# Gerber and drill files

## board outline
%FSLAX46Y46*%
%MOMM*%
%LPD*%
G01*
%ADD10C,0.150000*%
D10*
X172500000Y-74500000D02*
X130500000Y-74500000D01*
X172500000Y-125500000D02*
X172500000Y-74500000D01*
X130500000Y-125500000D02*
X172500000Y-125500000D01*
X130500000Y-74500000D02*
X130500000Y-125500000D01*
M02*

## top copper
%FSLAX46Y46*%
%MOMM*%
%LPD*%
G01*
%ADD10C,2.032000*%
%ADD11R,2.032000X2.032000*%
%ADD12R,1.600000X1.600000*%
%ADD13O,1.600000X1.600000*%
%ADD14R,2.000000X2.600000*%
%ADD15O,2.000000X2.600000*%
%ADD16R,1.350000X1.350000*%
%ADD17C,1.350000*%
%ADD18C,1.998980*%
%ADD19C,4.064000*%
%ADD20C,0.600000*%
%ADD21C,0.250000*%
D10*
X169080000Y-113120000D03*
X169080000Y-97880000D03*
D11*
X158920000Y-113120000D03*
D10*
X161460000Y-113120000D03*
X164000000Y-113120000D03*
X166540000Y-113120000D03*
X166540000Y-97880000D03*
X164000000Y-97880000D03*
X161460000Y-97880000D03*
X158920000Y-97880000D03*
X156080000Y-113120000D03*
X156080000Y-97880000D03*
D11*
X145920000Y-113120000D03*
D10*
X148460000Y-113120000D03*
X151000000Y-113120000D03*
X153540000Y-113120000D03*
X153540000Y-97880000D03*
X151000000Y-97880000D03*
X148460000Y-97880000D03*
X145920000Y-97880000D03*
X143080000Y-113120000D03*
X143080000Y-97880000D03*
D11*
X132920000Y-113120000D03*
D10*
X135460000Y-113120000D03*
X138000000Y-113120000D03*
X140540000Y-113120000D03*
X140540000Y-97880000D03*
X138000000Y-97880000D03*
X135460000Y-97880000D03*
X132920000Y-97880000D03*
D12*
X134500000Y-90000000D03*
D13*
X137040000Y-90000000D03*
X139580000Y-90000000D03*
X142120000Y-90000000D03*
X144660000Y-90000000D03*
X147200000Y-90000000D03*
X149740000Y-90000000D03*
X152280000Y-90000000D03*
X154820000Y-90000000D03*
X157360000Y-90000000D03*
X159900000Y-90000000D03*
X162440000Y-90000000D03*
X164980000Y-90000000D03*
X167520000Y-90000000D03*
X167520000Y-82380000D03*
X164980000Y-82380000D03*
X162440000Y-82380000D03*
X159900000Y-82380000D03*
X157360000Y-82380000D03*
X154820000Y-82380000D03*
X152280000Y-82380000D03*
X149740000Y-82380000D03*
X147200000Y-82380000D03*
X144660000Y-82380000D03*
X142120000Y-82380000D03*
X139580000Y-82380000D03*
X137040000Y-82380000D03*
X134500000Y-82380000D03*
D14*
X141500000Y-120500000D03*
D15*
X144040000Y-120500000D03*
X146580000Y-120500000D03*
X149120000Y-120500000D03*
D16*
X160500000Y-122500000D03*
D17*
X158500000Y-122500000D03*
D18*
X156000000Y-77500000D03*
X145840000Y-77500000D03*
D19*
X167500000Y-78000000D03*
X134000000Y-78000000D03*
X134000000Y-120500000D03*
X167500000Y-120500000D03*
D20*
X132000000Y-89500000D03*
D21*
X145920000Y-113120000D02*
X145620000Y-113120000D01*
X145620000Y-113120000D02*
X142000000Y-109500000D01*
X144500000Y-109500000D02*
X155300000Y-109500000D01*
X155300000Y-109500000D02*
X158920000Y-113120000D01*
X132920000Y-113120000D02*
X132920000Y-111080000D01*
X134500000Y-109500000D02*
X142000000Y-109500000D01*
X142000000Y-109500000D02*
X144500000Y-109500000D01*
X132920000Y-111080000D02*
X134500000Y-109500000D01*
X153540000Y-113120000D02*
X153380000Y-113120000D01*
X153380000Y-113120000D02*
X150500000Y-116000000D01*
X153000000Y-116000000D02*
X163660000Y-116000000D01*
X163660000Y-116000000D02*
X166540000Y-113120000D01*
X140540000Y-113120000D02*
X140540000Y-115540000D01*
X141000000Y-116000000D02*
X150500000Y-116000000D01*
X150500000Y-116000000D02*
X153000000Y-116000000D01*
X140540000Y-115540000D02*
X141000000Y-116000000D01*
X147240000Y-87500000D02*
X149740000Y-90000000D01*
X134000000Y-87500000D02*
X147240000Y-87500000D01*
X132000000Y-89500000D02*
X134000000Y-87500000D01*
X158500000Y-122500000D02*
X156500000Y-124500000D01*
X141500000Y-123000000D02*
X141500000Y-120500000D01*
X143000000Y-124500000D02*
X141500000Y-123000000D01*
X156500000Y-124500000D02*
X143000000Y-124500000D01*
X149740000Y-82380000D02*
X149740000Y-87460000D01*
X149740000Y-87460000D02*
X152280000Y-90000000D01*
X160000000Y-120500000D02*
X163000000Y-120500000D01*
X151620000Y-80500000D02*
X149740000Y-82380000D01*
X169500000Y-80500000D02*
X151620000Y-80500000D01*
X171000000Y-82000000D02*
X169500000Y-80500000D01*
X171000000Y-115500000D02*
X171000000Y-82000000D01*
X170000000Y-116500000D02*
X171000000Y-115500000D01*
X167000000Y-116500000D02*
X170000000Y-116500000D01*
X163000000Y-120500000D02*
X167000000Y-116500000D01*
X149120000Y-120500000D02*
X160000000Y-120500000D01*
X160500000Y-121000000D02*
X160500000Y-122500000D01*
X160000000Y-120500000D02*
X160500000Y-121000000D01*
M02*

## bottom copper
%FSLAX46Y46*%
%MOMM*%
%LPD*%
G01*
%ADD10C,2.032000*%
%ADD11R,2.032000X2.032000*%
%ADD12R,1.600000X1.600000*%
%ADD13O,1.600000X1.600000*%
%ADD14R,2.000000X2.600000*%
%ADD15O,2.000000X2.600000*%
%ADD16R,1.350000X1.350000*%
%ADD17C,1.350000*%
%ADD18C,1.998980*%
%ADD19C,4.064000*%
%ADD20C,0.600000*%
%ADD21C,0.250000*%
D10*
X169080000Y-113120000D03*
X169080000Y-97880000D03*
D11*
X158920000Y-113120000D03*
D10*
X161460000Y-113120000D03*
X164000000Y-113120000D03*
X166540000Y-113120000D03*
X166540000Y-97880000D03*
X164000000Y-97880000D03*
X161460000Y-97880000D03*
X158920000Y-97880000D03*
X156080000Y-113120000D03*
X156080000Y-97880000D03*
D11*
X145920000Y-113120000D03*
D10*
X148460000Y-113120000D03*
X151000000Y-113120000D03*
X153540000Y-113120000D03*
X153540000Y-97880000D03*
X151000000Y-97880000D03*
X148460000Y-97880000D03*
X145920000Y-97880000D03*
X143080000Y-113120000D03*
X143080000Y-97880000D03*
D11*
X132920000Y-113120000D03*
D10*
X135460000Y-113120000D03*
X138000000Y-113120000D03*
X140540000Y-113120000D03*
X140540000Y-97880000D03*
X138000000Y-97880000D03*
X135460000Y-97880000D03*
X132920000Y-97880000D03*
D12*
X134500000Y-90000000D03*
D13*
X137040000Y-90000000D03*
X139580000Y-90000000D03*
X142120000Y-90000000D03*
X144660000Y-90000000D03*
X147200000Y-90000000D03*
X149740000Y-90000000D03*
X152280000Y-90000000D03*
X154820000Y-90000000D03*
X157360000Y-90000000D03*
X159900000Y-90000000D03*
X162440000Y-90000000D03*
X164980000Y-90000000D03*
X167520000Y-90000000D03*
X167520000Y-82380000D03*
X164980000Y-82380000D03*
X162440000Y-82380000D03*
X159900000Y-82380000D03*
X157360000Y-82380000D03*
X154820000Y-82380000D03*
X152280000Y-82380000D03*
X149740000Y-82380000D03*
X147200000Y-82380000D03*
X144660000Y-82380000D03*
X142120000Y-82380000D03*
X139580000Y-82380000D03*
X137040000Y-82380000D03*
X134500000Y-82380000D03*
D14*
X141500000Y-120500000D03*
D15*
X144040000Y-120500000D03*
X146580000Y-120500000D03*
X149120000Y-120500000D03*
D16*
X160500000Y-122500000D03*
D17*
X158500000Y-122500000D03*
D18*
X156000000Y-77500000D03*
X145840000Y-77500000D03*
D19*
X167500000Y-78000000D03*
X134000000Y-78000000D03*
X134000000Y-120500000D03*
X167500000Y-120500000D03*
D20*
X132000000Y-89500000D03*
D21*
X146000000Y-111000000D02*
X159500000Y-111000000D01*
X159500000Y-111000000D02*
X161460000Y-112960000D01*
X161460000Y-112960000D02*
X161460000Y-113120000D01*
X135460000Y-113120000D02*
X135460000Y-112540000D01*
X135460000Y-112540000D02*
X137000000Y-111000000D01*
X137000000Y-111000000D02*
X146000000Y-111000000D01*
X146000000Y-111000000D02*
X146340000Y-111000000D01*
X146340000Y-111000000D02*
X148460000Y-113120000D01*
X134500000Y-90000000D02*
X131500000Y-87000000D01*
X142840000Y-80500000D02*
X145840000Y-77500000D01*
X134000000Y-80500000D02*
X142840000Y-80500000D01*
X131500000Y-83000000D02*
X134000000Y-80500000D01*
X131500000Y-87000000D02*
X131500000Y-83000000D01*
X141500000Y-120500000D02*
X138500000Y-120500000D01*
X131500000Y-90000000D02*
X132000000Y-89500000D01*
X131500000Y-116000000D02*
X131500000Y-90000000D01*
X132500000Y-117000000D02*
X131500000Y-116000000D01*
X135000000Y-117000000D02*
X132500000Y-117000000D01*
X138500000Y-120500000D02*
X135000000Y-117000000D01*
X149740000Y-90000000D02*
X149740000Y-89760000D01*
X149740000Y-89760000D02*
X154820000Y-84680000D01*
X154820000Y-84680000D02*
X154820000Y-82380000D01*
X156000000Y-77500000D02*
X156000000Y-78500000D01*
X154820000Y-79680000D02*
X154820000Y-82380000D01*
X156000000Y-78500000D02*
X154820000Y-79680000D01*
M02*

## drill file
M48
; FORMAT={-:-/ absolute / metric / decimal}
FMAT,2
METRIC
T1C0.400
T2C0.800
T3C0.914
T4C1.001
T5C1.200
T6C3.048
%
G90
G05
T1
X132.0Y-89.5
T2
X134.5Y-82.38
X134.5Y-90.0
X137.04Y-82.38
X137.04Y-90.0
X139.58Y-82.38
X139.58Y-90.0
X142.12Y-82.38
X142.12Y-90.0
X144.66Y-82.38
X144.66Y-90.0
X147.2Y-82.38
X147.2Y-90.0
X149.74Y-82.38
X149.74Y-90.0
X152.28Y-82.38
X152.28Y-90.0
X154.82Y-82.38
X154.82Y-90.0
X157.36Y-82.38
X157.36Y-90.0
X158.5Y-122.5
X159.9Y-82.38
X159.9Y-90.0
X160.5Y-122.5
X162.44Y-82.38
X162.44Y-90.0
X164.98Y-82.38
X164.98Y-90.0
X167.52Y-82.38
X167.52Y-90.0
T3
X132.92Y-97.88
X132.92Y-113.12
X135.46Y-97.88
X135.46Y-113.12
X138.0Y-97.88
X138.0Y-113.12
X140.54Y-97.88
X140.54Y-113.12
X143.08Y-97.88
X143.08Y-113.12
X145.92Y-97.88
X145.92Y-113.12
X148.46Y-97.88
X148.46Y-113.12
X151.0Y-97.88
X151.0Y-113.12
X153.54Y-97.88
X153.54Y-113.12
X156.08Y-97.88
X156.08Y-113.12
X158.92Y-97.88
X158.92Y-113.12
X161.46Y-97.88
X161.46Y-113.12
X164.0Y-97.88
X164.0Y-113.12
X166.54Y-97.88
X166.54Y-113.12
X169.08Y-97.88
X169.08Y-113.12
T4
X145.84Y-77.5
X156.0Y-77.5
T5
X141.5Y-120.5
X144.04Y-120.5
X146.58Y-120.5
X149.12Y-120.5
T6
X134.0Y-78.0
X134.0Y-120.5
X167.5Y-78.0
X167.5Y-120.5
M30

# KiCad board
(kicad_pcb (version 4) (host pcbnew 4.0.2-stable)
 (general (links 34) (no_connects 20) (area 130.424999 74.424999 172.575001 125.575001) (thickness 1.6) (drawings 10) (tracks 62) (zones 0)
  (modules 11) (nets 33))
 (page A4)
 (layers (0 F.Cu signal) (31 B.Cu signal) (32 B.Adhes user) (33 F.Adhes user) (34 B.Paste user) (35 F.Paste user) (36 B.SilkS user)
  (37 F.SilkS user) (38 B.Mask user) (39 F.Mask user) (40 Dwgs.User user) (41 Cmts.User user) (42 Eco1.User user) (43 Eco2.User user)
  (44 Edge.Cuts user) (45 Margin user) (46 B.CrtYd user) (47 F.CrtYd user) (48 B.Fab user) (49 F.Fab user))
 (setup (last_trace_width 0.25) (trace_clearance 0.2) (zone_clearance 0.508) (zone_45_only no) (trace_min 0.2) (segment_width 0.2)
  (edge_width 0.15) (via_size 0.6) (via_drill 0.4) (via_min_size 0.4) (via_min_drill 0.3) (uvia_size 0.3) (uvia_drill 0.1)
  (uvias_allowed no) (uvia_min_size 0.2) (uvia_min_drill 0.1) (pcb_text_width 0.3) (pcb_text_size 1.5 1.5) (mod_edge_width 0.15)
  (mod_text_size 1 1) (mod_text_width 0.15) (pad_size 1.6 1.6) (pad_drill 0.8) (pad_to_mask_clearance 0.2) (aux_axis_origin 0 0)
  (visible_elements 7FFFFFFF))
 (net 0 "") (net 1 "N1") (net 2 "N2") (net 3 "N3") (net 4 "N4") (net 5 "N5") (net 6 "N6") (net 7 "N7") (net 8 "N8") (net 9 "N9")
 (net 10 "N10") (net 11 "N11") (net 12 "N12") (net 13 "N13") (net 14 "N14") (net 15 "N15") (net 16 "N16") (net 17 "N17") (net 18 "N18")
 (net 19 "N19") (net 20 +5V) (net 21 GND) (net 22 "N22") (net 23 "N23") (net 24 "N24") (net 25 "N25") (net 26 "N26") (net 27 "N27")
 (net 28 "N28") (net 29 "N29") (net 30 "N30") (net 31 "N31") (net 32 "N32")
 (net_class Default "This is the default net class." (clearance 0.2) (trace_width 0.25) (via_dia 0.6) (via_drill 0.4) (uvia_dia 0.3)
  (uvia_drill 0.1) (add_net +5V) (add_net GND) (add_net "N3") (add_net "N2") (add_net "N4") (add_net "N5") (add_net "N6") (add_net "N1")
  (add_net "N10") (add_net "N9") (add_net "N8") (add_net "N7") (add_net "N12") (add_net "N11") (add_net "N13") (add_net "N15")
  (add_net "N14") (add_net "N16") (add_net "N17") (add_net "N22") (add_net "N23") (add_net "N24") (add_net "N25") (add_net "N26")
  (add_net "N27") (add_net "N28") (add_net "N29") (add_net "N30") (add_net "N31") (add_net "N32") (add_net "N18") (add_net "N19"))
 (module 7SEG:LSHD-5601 (layer F.Cu) (at 164 105.5)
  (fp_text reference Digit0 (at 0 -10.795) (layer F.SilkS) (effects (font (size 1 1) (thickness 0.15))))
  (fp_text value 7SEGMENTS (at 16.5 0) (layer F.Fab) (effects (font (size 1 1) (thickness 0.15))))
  (pad 5 thru_hole circle (at 5.08 7.62) (size 2.032 2.032) (drill 0.9144) (layers *.Cu *.Mask F.SilkS) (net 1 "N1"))
  (pad 10 thru_hole circle (at 5.08 -7.62) (size 2.032 2.032) (drill 0.9144) (layers *.Cu *.Mask F.SilkS) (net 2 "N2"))
  (pad 1 thru_hole rect (at -5.08 7.62) (size 2.032 2.032) (drill 0.9144) (layers *.Cu *.Mask F.SilkS) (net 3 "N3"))
  (pad 2 thru_hole circle (at -2.54 7.62) (size 2.032 2.032) (drill 0.9144) (layers *.Cu *.Mask F.SilkS) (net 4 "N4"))
  (pad 3 thru_hole circle (at 0 7.62) (size 2.032 2.032) (drill 0.9144) (layers *.Cu *.Mask F.SilkS) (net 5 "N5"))
  (pad 4 thru_hole circle (at 2.54 7.62) (size 2.032 2.032) (drill 0.9144) (layers *.Cu *.Mask F.SilkS) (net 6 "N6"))
  (pad 9 thru_hole circle (at 2.54 -7.62) (size 2.032 2.032) (drill 0.9144) (layers *.Cu *.Mask F.SilkS) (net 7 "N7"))
  (pad 8 thru_hole circle (at 0 -7.62) (size 2.032 2.032) (drill 0.9144) (layers *.Cu *.Mask F.SilkS) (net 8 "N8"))
  (pad 7 thru_hole circle (at -2.54 -7.62) (size 2.032 2.032) (drill 0.9144) (layers *.Cu *.Mask F.SilkS) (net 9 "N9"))
  (pad 6 thru_hole circle (at -5.08 -7.62) (size 2.032 2.032) (drill 0.9144) (layers *.Cu *.Mask F.SilkS) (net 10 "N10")))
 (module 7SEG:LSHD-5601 (layer F.Cu) (at 151 105.5)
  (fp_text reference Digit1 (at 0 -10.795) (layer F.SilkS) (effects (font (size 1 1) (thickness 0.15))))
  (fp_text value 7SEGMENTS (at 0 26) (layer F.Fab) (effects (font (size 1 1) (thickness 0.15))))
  (pad 5 thru_hole circle (at 5.08 7.62) (size 2.032 2.032) (drill 0.9144) (layers *.Cu *.Mask F.SilkS) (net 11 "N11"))
  (pad 10 thru_hole circle (at 5.08 -7.62) (size 2.032 2.032) (drill 0.9144) (layers *.Cu *.Mask F.SilkS) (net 2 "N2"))
  (pad 1 thru_hole rect (at -5.08 7.62) (size 2.032 2.032) (drill 0.9144) (layers *.Cu *.Mask F.SilkS) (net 3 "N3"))
  (pad 2 thru_hole circle (at -2.54 7.62) (size 2.032 2.032) (drill 0.9144) (layers *.Cu *.Mask F.SilkS) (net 4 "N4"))
  (pad 3 thru_hole circle (at 0 7.62) (size 2.032 2.032) (drill 0.9144) (layers *.Cu *.Mask F.SilkS) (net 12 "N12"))
  (pad 4 thru_hole circle (at 2.54 7.62) (size 2.032 2.032) (drill 0.9144) (layers *.Cu *.Mask F.SilkS) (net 6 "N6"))
  (pad 9 thru_hole circle (at 2.54 -7.62) (size 2.032 2.032) (drill 0.9144) (layers *.Cu *.Mask F.SilkS) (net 7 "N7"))
  (pad 8 thru_hole circle (at 0 -7.62) (size 2.032 2.032) (drill 0.9144) (layers *.Cu *.Mask F.SilkS) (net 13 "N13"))
  (pad 7 thru_hole circle (at -2.54 -7.62) (size 2.032 2.032) (drill 0.9144) (layers *.Cu *.Mask F.SilkS) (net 9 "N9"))
  (pad 6 thru_hole circle (at -5.08 -7.62) (size 2.032 2.032) (drill 0.9144) (layers *.Cu *.Mask F.SilkS) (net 10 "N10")))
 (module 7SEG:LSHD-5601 (layer F.Cu) (at 138 105.5)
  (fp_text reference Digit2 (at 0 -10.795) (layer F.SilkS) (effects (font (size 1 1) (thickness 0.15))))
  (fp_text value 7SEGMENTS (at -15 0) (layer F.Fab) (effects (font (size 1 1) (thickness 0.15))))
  (pad 5 thru_hole circle (at 5.08 7.62) (size 2.032 2.032) (drill 0.9144) (layers *.Cu *.Mask F.SilkS) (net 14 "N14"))
  (pad 10 thru_hole circle (at 5.08 -7.62) (size 2.032 2.032) (drill 0.9144) (layers *.Cu *.Mask F.SilkS) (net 2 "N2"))
  (pad 1 thru_hole rect (at -5.08 7.62) (size 2.032 2.032) (drill 0.9144) (layers *.Cu *.Mask F.SilkS) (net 3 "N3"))
  (pad 2 thru_hole circle (at -2.54 7.62) (size 2.032 2.032) (drill 0.9144) (layers *.Cu *.Mask F.SilkS) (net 4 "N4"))
  (pad 3 thru_hole circle (at 0 7.62) (size 2.032 2.032) (drill 0.9144) (layers *.Cu *.Mask F.SilkS) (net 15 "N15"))
  (pad 4 thru_hole circle (at 2.54 7.62) (size 2.032 2.032) (drill 0.9144) (layers *.Cu *.Mask F.SilkS) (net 6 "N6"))
  (pad 9 thru_hole circle (at 2.54 -7.62) (size 2.032 2.032) (drill 0.9144) (layers *.Cu *.Mask F.SilkS) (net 7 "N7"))
  (pad 8 thru_hole circle (at 0 -7.62) (size 2.032 2.032) (drill 0.9144) (layers *.Cu *.Mask F.SilkS) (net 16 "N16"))
  (pad 7 thru_hole circle (at -2.54 -7.62) (size 2.032 2.032) (drill 0.9144) (layers *.Cu *.Mask F.SilkS) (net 9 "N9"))
  (pad 6 thru_hole circle (at -5.08 -7.62) (size 2.032 2.032) (drill 0.9144) (layers *.Cu *.Mask F.SilkS) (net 10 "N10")))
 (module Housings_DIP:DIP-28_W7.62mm (layer F.Cu) (at 134.5 90 90)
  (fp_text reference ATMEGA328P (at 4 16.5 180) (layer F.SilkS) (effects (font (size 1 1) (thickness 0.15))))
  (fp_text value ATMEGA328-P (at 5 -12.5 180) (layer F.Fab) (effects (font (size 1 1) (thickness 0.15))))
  (pad 1 thru_hole rect (at 0 0 90) (size 1.6 1.6) (drill 0.8) (layers *.Cu *.Mask F.SilkS) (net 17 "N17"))
  (pad 2 thru_hole oval (at 0 2.54 90) (size 1.6 1.6) (drill 0.8) (layers *.Cu *.Mask F.SilkS) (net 8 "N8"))
  (pad 3 thru_hole oval (at 0 5.08 90) (size 1.6 1.6) (drill 0.8) (layers *.Cu *.Mask F.SilkS) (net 13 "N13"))
  (pad 4 thru_hole oval (at 0 7.62 90) (size 1.6 1.6) (drill 0.8) (layers *.Cu *.Mask F.SilkS) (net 16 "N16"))
  (pad 5 thru_hole oval (at 0 10.16 90) (size 1.6 1.6) (drill 0.8) (layers *.Cu *.Mask F.SilkS) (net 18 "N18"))
  (pad 6 thru_hole oval (at 0 12.7 90) (size 1.6 1.6) (drill 0.8) (layers *.Cu *.Mask F.SilkS) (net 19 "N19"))
  (pad 7 thru_hole oval (at 0 15.24 90) (size 1.6 1.6) (drill 0.8) (layers *.Cu *.Mask F.SilkS) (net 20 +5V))
  (pad 8 thru_hole oval (at 0 17.78 90) (size 1.6 1.6) (drill 0.8) (layers *.Cu *.Mask F.SilkS) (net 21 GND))
  (pad 9 thru_hole oval (at 0 20.32 90) (size 1.6 1.6) (drill 0.8) (layers *.Cu *.Mask F.SilkS) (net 2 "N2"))
  (pad 10 thru_hole oval (at 0 22.86 90) (size 1.6 1.6) (drill 0.8) (layers *.Cu *.Mask F.SilkS) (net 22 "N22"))
  (pad 11 thru_hole oval (at 0 25.4 90) (size 1.6 1.6) (drill 0.8) (layers *.Cu *.Mask F.SilkS) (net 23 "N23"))
  (pad 12 thru_hole oval (at 0 27.94 90) (size 1.6 1.6) (drill 0.8) (layers *.Cu *.Mask F.SilkS) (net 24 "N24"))
  (pad 13 thru_hole oval (at 0 30.48 90) (size 1.6 1.6) (drill 0.8) (layers *.Cu *.Mask F.SilkS) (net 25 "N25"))
  (pad 14 thru_hole oval (at 0 33.02 90) (size 1.6 1.6) (drill 0.8) (layers *.Cu *.Mask F.SilkS) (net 9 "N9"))
  (pad 15 thru_hole oval (at 7.62 33.02 90) (size 1.6 1.6) (drill 0.8) (layers *.Cu *.Mask F.SilkS) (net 10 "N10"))
  (pad 16 thru_hole oval (at 7.62 30.48 90) (size 1.6 1.6) (drill 0.8) (layers *.Cu *.Mask F.SilkS) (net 6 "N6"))
  (pad 17 thru_hole oval (at 7.62 27.94 90) (size 1.6 1.6) (drill 0.8) (layers *.Cu *.Mask F.SilkS) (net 4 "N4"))
  (pad 18 thru_hole oval (at 7.62 25.4 90) (size 1.6 1.6) (drill 0.8) (layers *.Cu *.Mask F.SilkS) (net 3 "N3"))
  (pad 19 thru_hole oval (at 7.62 22.86 90) (size 1.6 1.6) (drill 0.8) (layers *.Cu *.Mask F.SilkS) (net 7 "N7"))
  (pad 20 thru_hole oval (at 7.62 20.32 90) (size 1.6 1.6) (drill 0.8) (layers *.Cu *.Mask F.SilkS) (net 20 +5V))
  (pad 21 thru_hole oval (at 7.62 17.78 90) (size 1.6 1.6) (drill 0.8) (layers *.Cu *.Mask F.SilkS) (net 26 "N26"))
  (pad 22 thru_hole oval (at 7.62 15.24 90) (size 1.6 1.6) (drill 0.8) (layers *.Cu *.Mask F.SilkS) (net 21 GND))
  (pad 23 thru_hole oval (at 7.62 12.7 90) (size 1.6 1.6) (drill 0.8) (layers *.Cu *.Mask F.SilkS) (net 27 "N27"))
  (pad 24 thru_hole oval (at 7.62 10.16 90) (size 1.6 1.6) (drill 0.8) (layers *.Cu *.Mask F.SilkS) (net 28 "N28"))
  (pad 25 thru_hole oval (at 7.62 7.62 90) (size 1.6 1.6) (drill 0.8) (layers *.Cu *.Mask F.SilkS) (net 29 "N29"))
  (pad 26 thru_hole oval (at 7.62 5.08 90) (size 1.6 1.6) (drill 0.8) (layers *.Cu *.Mask F.SilkS) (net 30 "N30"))
  (pad 27 thru_hole oval (at 7.62 2.54 90) (size 1.6 1.6) (drill 0.8) (layers *.Cu *.Mask F.SilkS) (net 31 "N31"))
  (pad 28 thru_hole oval (at 7.62 0 90) (size 1.6 1.6) (drill 0.8) (layers *.Cu *.Mask F.SilkS) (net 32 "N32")))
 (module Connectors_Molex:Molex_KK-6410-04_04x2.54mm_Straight (layer F.Cu) (at 141.5 120.5)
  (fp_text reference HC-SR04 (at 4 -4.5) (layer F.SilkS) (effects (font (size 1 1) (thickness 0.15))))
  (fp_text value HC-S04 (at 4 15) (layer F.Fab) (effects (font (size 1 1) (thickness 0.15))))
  (pad 1 thru_hole rect (at 0 0) (size 2 2.6) (drill 1.2) (layers *.Cu *.Mask F.SilkS) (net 20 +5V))
  (pad 2 thru_hole oval (at 2.54 0) (size 2 2.6) (drill 1.2) (layers *.Cu *.Mask F.SilkS) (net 18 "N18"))
  (pad 3 thru_hole oval (at 5.08 0) (size 2 2.6) (drill 1.2) (layers *.Cu *.Mask F.SilkS) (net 19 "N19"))
  (pad 4 thru_hole oval (at 7.62 0) (size 2 2.6) (drill 1.2) (layers *.Cu *.Mask F.SilkS) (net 21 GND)))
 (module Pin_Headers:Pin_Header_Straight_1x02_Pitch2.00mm (layer F.Cu) (at 160.5 122.5 270)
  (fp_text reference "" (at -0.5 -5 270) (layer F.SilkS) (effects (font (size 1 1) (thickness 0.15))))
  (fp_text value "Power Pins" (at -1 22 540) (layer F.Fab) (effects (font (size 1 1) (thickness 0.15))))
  (pad 1 thru_hole rect (at 0 0 270) (size 1.35 1.35) (drill 0.8) (layers *.Cu *.Mask) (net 21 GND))
  (pad 2 thru_hole circle (at 0 2 270) (size 1.35 1.35) (drill 0.8) (layers *.Cu *.Mask) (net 20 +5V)))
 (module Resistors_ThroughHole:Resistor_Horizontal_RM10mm (layer F.Cu) (at 156 77.5 180)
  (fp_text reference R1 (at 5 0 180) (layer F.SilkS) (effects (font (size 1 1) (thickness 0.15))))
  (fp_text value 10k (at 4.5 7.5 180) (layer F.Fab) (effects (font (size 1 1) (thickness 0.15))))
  (pad 1 thru_hole circle (at 0 0 180) (size 1.99898 1.99898) (drill 1.00076) (layers *.Cu *.SilkS *.Mask) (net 20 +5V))
  (pad 2 thru_hole circle (at 10.16 0 180) (size 1.99898 1.99898) (drill 1.00076) (layers *.Cu *.SilkS *.Mask) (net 17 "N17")))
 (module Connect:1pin (layer F.Cu) (at 167.5 78)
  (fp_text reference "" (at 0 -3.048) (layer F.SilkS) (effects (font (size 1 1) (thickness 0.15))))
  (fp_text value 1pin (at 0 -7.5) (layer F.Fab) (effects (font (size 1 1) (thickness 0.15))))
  (pad 1 thru_hole circle (at 0 0) (size 4.064 4.064) (drill 3.048) (layers *.Cu *.Mask F.SilkS)))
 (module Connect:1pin (layer F.Cu) (at 134 78)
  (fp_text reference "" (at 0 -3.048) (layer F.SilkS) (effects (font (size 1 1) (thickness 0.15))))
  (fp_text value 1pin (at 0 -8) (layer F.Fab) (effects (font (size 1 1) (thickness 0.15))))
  (pad 1 thru_hole circle (at 0 0) (size 4.064 4.064) (drill 3.048) (layers *.Cu *.Mask F.SilkS)))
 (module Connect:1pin (layer F.Cu) (at 134 120.5)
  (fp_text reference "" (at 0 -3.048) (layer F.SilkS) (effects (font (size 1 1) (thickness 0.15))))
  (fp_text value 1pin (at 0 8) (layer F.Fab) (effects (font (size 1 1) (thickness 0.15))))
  (pad 1 thru_hole circle (at 0 0) (size 4.064 4.064) (drill 3.048) (layers *.Cu *.Mask F.SilkS)))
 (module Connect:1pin (layer F.Cu) (at 167.5 120.5)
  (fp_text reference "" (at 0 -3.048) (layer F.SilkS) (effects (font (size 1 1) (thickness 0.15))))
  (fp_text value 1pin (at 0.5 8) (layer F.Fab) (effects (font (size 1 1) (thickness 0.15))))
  (pad 1 thru_hole circle (at 0 0) (size 4.064 4.064) (drill 3.048) (layers *.Cu *.Mask F.SilkS)))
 (gr_line (start 172.5 74.5) (end 130.5 74.5) (angle 90) (layer Edge.Cuts) (width 0.15))
 (gr_line (start 172.5 125.5) (end 172.5 74.5) (angle 90) (layer Edge.Cuts) (width 0.15))
 (gr_line (start 130.5 125.5) (end 172.5 125.5) (angle 90) (layer Edge.Cuts) (width 0.15))
 (gr_line (start 130.5 74.5) (end 130.5 125.5) (angle 90) (layer Edge.Cuts) (width 0.15))
 (segment (start 145.92 113.12) (end 145.62 113.12) (width 0.25) (layer F.Cu) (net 3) (status C00000))
 (segment (start 145.62 113.12) (end 142 109.5) (width 0.25) (layer F.Cu) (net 3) (status 400000))
 (segment (start 144.5 109.5) (end 155.3 109.5) (width 0.25) (layer F.Cu) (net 3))
 (segment (start 155.3 109.5) (end 158.92 113.12) (width 0.25) (layer F.Cu) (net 3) (status 800000))
 (segment (start 132.92 113.12) (end 132.92 111.08) (width 0.25) (layer F.Cu) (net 3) (status 400000))
 (segment (start 134.5 109.5) (end 142 109.5) (width 0.25) (layer F.Cu) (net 3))
 (segment (start 142 109.5) (end 144.5 109.5) (width 0.25) (layer F.Cu) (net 3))
 (segment (start 132.92 111.08) (end 134.5 109.5) (width 0.25) (layer F.Cu) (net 3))
 (segment (start 146 111) (end 159.5 111) (width 0.25) (layer B.Cu) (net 4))
 (segment (start 159.5 111) (end 161.46 112.96) (width 0.25) (layer B.Cu) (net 4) (status 800000))
 (segment (start 161.46 112.96) (end 161.46 113.12) (width 0.25) (layer B.Cu) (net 4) (status C00000))
 (segment (start 135.46 113.12) (end 135.46 112.54) (width 0.25) (layer B.Cu) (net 4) (status C00000))
 (segment (start 135.46 112.54) (end 137 111) (width 0.25) (layer B.Cu) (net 4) (status 400000))
 (segment (start 137 111) (end 146 111) (width 0.25) (layer B.Cu) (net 4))
 (segment (start 146 111) (end 146.34 111) (width 0.25) (layer B.Cu) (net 4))
 (segment (start 146.34 111) (end 148.46 113.12) (width 0.25) (layer B.Cu) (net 4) (status 800000))
 (segment (start 153.54 113.12) (end 153.38 113.12) (width 0.25) (layer F.Cu) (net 6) (status C00000))
 (segment (start 153.38 113.12) (end 150.5 116) (width 0.25) (layer F.Cu) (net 6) (status 400000))
 (segment (start 153 116) (end 163.66 116) (width 0.25) (layer F.Cu) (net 6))
 (segment (start 163.66 116) (end 166.54 113.12) (width 0.25) (layer F.Cu) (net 6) (status 800000))
 (segment (start 140.54 113.12) (end 140.54 115.54) (width 0.25) (layer F.Cu) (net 6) (status 400000))
 (segment (start 141 116) (end 150.5 116) (width 0.25) (layer F.Cu) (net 6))
 (segment (start 150.5 116) (end 153 116) (width 0.25) (layer F.Cu) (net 6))
 (segment (start 140.54 115.54) (end 141 116) (width 0.25) (layer F.Cu) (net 6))
 (segment (start 134.5 90) (end 131.5 87) (width 0.25) (layer B.Cu) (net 17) (status 400000))
 (segment (start 142.84 80.5) (end 145.84 77.5) (width 0.25) (layer B.Cu) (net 17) (status 800000))
 (segment (start 134 80.5) (end 142.84 80.5) (width 0.25) (layer B.Cu) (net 17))
 (segment (start 131.5 83) (end 134 80.5) (width 0.25) (layer B.Cu) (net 17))
 (segment (start 131.5 87) (end 131.5 83) (width 0.25) (layer B.Cu) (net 17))
 (segment (start 141.5 120.5) (end 138.5 120.5) (width 0.25) (layer B.Cu) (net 20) (status 400000))
 (segment (start 147.24 87.5) (end 149.74 90) (width 0.25) (layer F.Cu) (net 20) (status 800000))
 (segment (start 134 87.5) (end 147.24 87.5) (width 0.25) (layer F.Cu) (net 20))
 (segment (start 132 89.5) (end 134 87.5) (width 0.25) (layer F.Cu) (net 20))
 (via (at 132 89.5) (size 0.6) (drill 0.4) (layers F.Cu B.Cu) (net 20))
 (segment (start 131.5 90) (end 132 89.5) (width 0.25) (layer B.Cu) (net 20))
 (segment (start 131.5 116) (end 131.5 90) (width 0.25) (layer B.Cu) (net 20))
 (segment (start 132.5 117) (end 131.5 116) (width 0.25) (layer B.Cu) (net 20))
 (segment (start 135 117) (end 132.5 117) (width 0.25) (layer B.Cu) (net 20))
 (segment (start 138.5 120.5) (end 135 117) (width 0.25) (layer B.Cu) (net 20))
 (segment (start 149.74 90) (end 149.74 89.76) (width 0.25) (layer B.Cu) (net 20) (status C00000))
 (segment (start 149.74 89.76) (end 154.82 84.68) (width 0.25) (layer B.Cu) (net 20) (status 400000))
 (segment (start 154.82 84.68) (end 154.82 82.38) (width 0.25) (layer B.Cu) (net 20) (status 800000))
 (segment (start 156 77.5) (end 156 78.5) (width 0.25) (layer B.Cu) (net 20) (status 400000))
 (segment (start 154.82 79.68) (end 154.82 82.38) (width 0.25) (layer B.Cu) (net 20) (status 800000))
 (segment (start 156 78.5) (end 154.82 79.68) (width 0.25) (layer B.Cu) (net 20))
 (segment (start 158.5 122.5) (end 156.5 124.5) (width 0.25) (layer F.Cu) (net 20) (status 400000))
 (segment (start 141.5 123) (end 141.5 120.5) (width 0.25) (layer F.Cu) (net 20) (status 800000))
 (segment (start 143 124.5) (end 141.5 123) (width 0.25) (layer F.Cu) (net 20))
 (segment (start 156.5 124.5) (end 143 124.5) (width 0.25) (layer F.Cu) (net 20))
 (segment (start 149.74 82.38) (end 149.74 87.46) (width 0.25) (layer F.Cu) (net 21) (status 400000))
 (segment (start 149.74 87.46) (end 152.28 90) (width 0.25) (layer F.Cu) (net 21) (status 800000))
 (segment (start 160 120.5) (end 163 120.5) (width 0.25) (layer F.Cu) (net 21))
 (segment (start 151.62 80.5) (end 149.74 82.38) (width 0.25) (layer F.Cu) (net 21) (status 800000))
 (segment (start 169.5 80.5) (end 151.62 80.5) (width 0.25) (layer F.Cu) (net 21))
 (segment (start 171 82) (end 169.5 80.5) (width 0.25) (layer F.Cu) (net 21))
 (segment (start 171 115.5) (end 171 82) (width 0.25) (layer F.Cu) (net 21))
 (segment (start 170 116.5) (end 171 115.5) (width 0.25) (layer F.Cu) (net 21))
 (segment (start 167 116.5) (end 170 116.5) (width 0.25) (layer F.Cu) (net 21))
 (segment (start 163 120.5) (end 167 116.5) (width 0.25) (layer F.Cu) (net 21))
 (segment (start 149.12 120.5) (end 160 120.5) (width 0.25) (layer F.Cu) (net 21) (status 400000))
 (segment (start 160.5 121) (end 160.5 122.5) (width 0.25) (layer F.Cu) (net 21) (status 800000))
 (segment (start 160 120.5) (end 160.5 121) (width 0.25) (layer F.Cu) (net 21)))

